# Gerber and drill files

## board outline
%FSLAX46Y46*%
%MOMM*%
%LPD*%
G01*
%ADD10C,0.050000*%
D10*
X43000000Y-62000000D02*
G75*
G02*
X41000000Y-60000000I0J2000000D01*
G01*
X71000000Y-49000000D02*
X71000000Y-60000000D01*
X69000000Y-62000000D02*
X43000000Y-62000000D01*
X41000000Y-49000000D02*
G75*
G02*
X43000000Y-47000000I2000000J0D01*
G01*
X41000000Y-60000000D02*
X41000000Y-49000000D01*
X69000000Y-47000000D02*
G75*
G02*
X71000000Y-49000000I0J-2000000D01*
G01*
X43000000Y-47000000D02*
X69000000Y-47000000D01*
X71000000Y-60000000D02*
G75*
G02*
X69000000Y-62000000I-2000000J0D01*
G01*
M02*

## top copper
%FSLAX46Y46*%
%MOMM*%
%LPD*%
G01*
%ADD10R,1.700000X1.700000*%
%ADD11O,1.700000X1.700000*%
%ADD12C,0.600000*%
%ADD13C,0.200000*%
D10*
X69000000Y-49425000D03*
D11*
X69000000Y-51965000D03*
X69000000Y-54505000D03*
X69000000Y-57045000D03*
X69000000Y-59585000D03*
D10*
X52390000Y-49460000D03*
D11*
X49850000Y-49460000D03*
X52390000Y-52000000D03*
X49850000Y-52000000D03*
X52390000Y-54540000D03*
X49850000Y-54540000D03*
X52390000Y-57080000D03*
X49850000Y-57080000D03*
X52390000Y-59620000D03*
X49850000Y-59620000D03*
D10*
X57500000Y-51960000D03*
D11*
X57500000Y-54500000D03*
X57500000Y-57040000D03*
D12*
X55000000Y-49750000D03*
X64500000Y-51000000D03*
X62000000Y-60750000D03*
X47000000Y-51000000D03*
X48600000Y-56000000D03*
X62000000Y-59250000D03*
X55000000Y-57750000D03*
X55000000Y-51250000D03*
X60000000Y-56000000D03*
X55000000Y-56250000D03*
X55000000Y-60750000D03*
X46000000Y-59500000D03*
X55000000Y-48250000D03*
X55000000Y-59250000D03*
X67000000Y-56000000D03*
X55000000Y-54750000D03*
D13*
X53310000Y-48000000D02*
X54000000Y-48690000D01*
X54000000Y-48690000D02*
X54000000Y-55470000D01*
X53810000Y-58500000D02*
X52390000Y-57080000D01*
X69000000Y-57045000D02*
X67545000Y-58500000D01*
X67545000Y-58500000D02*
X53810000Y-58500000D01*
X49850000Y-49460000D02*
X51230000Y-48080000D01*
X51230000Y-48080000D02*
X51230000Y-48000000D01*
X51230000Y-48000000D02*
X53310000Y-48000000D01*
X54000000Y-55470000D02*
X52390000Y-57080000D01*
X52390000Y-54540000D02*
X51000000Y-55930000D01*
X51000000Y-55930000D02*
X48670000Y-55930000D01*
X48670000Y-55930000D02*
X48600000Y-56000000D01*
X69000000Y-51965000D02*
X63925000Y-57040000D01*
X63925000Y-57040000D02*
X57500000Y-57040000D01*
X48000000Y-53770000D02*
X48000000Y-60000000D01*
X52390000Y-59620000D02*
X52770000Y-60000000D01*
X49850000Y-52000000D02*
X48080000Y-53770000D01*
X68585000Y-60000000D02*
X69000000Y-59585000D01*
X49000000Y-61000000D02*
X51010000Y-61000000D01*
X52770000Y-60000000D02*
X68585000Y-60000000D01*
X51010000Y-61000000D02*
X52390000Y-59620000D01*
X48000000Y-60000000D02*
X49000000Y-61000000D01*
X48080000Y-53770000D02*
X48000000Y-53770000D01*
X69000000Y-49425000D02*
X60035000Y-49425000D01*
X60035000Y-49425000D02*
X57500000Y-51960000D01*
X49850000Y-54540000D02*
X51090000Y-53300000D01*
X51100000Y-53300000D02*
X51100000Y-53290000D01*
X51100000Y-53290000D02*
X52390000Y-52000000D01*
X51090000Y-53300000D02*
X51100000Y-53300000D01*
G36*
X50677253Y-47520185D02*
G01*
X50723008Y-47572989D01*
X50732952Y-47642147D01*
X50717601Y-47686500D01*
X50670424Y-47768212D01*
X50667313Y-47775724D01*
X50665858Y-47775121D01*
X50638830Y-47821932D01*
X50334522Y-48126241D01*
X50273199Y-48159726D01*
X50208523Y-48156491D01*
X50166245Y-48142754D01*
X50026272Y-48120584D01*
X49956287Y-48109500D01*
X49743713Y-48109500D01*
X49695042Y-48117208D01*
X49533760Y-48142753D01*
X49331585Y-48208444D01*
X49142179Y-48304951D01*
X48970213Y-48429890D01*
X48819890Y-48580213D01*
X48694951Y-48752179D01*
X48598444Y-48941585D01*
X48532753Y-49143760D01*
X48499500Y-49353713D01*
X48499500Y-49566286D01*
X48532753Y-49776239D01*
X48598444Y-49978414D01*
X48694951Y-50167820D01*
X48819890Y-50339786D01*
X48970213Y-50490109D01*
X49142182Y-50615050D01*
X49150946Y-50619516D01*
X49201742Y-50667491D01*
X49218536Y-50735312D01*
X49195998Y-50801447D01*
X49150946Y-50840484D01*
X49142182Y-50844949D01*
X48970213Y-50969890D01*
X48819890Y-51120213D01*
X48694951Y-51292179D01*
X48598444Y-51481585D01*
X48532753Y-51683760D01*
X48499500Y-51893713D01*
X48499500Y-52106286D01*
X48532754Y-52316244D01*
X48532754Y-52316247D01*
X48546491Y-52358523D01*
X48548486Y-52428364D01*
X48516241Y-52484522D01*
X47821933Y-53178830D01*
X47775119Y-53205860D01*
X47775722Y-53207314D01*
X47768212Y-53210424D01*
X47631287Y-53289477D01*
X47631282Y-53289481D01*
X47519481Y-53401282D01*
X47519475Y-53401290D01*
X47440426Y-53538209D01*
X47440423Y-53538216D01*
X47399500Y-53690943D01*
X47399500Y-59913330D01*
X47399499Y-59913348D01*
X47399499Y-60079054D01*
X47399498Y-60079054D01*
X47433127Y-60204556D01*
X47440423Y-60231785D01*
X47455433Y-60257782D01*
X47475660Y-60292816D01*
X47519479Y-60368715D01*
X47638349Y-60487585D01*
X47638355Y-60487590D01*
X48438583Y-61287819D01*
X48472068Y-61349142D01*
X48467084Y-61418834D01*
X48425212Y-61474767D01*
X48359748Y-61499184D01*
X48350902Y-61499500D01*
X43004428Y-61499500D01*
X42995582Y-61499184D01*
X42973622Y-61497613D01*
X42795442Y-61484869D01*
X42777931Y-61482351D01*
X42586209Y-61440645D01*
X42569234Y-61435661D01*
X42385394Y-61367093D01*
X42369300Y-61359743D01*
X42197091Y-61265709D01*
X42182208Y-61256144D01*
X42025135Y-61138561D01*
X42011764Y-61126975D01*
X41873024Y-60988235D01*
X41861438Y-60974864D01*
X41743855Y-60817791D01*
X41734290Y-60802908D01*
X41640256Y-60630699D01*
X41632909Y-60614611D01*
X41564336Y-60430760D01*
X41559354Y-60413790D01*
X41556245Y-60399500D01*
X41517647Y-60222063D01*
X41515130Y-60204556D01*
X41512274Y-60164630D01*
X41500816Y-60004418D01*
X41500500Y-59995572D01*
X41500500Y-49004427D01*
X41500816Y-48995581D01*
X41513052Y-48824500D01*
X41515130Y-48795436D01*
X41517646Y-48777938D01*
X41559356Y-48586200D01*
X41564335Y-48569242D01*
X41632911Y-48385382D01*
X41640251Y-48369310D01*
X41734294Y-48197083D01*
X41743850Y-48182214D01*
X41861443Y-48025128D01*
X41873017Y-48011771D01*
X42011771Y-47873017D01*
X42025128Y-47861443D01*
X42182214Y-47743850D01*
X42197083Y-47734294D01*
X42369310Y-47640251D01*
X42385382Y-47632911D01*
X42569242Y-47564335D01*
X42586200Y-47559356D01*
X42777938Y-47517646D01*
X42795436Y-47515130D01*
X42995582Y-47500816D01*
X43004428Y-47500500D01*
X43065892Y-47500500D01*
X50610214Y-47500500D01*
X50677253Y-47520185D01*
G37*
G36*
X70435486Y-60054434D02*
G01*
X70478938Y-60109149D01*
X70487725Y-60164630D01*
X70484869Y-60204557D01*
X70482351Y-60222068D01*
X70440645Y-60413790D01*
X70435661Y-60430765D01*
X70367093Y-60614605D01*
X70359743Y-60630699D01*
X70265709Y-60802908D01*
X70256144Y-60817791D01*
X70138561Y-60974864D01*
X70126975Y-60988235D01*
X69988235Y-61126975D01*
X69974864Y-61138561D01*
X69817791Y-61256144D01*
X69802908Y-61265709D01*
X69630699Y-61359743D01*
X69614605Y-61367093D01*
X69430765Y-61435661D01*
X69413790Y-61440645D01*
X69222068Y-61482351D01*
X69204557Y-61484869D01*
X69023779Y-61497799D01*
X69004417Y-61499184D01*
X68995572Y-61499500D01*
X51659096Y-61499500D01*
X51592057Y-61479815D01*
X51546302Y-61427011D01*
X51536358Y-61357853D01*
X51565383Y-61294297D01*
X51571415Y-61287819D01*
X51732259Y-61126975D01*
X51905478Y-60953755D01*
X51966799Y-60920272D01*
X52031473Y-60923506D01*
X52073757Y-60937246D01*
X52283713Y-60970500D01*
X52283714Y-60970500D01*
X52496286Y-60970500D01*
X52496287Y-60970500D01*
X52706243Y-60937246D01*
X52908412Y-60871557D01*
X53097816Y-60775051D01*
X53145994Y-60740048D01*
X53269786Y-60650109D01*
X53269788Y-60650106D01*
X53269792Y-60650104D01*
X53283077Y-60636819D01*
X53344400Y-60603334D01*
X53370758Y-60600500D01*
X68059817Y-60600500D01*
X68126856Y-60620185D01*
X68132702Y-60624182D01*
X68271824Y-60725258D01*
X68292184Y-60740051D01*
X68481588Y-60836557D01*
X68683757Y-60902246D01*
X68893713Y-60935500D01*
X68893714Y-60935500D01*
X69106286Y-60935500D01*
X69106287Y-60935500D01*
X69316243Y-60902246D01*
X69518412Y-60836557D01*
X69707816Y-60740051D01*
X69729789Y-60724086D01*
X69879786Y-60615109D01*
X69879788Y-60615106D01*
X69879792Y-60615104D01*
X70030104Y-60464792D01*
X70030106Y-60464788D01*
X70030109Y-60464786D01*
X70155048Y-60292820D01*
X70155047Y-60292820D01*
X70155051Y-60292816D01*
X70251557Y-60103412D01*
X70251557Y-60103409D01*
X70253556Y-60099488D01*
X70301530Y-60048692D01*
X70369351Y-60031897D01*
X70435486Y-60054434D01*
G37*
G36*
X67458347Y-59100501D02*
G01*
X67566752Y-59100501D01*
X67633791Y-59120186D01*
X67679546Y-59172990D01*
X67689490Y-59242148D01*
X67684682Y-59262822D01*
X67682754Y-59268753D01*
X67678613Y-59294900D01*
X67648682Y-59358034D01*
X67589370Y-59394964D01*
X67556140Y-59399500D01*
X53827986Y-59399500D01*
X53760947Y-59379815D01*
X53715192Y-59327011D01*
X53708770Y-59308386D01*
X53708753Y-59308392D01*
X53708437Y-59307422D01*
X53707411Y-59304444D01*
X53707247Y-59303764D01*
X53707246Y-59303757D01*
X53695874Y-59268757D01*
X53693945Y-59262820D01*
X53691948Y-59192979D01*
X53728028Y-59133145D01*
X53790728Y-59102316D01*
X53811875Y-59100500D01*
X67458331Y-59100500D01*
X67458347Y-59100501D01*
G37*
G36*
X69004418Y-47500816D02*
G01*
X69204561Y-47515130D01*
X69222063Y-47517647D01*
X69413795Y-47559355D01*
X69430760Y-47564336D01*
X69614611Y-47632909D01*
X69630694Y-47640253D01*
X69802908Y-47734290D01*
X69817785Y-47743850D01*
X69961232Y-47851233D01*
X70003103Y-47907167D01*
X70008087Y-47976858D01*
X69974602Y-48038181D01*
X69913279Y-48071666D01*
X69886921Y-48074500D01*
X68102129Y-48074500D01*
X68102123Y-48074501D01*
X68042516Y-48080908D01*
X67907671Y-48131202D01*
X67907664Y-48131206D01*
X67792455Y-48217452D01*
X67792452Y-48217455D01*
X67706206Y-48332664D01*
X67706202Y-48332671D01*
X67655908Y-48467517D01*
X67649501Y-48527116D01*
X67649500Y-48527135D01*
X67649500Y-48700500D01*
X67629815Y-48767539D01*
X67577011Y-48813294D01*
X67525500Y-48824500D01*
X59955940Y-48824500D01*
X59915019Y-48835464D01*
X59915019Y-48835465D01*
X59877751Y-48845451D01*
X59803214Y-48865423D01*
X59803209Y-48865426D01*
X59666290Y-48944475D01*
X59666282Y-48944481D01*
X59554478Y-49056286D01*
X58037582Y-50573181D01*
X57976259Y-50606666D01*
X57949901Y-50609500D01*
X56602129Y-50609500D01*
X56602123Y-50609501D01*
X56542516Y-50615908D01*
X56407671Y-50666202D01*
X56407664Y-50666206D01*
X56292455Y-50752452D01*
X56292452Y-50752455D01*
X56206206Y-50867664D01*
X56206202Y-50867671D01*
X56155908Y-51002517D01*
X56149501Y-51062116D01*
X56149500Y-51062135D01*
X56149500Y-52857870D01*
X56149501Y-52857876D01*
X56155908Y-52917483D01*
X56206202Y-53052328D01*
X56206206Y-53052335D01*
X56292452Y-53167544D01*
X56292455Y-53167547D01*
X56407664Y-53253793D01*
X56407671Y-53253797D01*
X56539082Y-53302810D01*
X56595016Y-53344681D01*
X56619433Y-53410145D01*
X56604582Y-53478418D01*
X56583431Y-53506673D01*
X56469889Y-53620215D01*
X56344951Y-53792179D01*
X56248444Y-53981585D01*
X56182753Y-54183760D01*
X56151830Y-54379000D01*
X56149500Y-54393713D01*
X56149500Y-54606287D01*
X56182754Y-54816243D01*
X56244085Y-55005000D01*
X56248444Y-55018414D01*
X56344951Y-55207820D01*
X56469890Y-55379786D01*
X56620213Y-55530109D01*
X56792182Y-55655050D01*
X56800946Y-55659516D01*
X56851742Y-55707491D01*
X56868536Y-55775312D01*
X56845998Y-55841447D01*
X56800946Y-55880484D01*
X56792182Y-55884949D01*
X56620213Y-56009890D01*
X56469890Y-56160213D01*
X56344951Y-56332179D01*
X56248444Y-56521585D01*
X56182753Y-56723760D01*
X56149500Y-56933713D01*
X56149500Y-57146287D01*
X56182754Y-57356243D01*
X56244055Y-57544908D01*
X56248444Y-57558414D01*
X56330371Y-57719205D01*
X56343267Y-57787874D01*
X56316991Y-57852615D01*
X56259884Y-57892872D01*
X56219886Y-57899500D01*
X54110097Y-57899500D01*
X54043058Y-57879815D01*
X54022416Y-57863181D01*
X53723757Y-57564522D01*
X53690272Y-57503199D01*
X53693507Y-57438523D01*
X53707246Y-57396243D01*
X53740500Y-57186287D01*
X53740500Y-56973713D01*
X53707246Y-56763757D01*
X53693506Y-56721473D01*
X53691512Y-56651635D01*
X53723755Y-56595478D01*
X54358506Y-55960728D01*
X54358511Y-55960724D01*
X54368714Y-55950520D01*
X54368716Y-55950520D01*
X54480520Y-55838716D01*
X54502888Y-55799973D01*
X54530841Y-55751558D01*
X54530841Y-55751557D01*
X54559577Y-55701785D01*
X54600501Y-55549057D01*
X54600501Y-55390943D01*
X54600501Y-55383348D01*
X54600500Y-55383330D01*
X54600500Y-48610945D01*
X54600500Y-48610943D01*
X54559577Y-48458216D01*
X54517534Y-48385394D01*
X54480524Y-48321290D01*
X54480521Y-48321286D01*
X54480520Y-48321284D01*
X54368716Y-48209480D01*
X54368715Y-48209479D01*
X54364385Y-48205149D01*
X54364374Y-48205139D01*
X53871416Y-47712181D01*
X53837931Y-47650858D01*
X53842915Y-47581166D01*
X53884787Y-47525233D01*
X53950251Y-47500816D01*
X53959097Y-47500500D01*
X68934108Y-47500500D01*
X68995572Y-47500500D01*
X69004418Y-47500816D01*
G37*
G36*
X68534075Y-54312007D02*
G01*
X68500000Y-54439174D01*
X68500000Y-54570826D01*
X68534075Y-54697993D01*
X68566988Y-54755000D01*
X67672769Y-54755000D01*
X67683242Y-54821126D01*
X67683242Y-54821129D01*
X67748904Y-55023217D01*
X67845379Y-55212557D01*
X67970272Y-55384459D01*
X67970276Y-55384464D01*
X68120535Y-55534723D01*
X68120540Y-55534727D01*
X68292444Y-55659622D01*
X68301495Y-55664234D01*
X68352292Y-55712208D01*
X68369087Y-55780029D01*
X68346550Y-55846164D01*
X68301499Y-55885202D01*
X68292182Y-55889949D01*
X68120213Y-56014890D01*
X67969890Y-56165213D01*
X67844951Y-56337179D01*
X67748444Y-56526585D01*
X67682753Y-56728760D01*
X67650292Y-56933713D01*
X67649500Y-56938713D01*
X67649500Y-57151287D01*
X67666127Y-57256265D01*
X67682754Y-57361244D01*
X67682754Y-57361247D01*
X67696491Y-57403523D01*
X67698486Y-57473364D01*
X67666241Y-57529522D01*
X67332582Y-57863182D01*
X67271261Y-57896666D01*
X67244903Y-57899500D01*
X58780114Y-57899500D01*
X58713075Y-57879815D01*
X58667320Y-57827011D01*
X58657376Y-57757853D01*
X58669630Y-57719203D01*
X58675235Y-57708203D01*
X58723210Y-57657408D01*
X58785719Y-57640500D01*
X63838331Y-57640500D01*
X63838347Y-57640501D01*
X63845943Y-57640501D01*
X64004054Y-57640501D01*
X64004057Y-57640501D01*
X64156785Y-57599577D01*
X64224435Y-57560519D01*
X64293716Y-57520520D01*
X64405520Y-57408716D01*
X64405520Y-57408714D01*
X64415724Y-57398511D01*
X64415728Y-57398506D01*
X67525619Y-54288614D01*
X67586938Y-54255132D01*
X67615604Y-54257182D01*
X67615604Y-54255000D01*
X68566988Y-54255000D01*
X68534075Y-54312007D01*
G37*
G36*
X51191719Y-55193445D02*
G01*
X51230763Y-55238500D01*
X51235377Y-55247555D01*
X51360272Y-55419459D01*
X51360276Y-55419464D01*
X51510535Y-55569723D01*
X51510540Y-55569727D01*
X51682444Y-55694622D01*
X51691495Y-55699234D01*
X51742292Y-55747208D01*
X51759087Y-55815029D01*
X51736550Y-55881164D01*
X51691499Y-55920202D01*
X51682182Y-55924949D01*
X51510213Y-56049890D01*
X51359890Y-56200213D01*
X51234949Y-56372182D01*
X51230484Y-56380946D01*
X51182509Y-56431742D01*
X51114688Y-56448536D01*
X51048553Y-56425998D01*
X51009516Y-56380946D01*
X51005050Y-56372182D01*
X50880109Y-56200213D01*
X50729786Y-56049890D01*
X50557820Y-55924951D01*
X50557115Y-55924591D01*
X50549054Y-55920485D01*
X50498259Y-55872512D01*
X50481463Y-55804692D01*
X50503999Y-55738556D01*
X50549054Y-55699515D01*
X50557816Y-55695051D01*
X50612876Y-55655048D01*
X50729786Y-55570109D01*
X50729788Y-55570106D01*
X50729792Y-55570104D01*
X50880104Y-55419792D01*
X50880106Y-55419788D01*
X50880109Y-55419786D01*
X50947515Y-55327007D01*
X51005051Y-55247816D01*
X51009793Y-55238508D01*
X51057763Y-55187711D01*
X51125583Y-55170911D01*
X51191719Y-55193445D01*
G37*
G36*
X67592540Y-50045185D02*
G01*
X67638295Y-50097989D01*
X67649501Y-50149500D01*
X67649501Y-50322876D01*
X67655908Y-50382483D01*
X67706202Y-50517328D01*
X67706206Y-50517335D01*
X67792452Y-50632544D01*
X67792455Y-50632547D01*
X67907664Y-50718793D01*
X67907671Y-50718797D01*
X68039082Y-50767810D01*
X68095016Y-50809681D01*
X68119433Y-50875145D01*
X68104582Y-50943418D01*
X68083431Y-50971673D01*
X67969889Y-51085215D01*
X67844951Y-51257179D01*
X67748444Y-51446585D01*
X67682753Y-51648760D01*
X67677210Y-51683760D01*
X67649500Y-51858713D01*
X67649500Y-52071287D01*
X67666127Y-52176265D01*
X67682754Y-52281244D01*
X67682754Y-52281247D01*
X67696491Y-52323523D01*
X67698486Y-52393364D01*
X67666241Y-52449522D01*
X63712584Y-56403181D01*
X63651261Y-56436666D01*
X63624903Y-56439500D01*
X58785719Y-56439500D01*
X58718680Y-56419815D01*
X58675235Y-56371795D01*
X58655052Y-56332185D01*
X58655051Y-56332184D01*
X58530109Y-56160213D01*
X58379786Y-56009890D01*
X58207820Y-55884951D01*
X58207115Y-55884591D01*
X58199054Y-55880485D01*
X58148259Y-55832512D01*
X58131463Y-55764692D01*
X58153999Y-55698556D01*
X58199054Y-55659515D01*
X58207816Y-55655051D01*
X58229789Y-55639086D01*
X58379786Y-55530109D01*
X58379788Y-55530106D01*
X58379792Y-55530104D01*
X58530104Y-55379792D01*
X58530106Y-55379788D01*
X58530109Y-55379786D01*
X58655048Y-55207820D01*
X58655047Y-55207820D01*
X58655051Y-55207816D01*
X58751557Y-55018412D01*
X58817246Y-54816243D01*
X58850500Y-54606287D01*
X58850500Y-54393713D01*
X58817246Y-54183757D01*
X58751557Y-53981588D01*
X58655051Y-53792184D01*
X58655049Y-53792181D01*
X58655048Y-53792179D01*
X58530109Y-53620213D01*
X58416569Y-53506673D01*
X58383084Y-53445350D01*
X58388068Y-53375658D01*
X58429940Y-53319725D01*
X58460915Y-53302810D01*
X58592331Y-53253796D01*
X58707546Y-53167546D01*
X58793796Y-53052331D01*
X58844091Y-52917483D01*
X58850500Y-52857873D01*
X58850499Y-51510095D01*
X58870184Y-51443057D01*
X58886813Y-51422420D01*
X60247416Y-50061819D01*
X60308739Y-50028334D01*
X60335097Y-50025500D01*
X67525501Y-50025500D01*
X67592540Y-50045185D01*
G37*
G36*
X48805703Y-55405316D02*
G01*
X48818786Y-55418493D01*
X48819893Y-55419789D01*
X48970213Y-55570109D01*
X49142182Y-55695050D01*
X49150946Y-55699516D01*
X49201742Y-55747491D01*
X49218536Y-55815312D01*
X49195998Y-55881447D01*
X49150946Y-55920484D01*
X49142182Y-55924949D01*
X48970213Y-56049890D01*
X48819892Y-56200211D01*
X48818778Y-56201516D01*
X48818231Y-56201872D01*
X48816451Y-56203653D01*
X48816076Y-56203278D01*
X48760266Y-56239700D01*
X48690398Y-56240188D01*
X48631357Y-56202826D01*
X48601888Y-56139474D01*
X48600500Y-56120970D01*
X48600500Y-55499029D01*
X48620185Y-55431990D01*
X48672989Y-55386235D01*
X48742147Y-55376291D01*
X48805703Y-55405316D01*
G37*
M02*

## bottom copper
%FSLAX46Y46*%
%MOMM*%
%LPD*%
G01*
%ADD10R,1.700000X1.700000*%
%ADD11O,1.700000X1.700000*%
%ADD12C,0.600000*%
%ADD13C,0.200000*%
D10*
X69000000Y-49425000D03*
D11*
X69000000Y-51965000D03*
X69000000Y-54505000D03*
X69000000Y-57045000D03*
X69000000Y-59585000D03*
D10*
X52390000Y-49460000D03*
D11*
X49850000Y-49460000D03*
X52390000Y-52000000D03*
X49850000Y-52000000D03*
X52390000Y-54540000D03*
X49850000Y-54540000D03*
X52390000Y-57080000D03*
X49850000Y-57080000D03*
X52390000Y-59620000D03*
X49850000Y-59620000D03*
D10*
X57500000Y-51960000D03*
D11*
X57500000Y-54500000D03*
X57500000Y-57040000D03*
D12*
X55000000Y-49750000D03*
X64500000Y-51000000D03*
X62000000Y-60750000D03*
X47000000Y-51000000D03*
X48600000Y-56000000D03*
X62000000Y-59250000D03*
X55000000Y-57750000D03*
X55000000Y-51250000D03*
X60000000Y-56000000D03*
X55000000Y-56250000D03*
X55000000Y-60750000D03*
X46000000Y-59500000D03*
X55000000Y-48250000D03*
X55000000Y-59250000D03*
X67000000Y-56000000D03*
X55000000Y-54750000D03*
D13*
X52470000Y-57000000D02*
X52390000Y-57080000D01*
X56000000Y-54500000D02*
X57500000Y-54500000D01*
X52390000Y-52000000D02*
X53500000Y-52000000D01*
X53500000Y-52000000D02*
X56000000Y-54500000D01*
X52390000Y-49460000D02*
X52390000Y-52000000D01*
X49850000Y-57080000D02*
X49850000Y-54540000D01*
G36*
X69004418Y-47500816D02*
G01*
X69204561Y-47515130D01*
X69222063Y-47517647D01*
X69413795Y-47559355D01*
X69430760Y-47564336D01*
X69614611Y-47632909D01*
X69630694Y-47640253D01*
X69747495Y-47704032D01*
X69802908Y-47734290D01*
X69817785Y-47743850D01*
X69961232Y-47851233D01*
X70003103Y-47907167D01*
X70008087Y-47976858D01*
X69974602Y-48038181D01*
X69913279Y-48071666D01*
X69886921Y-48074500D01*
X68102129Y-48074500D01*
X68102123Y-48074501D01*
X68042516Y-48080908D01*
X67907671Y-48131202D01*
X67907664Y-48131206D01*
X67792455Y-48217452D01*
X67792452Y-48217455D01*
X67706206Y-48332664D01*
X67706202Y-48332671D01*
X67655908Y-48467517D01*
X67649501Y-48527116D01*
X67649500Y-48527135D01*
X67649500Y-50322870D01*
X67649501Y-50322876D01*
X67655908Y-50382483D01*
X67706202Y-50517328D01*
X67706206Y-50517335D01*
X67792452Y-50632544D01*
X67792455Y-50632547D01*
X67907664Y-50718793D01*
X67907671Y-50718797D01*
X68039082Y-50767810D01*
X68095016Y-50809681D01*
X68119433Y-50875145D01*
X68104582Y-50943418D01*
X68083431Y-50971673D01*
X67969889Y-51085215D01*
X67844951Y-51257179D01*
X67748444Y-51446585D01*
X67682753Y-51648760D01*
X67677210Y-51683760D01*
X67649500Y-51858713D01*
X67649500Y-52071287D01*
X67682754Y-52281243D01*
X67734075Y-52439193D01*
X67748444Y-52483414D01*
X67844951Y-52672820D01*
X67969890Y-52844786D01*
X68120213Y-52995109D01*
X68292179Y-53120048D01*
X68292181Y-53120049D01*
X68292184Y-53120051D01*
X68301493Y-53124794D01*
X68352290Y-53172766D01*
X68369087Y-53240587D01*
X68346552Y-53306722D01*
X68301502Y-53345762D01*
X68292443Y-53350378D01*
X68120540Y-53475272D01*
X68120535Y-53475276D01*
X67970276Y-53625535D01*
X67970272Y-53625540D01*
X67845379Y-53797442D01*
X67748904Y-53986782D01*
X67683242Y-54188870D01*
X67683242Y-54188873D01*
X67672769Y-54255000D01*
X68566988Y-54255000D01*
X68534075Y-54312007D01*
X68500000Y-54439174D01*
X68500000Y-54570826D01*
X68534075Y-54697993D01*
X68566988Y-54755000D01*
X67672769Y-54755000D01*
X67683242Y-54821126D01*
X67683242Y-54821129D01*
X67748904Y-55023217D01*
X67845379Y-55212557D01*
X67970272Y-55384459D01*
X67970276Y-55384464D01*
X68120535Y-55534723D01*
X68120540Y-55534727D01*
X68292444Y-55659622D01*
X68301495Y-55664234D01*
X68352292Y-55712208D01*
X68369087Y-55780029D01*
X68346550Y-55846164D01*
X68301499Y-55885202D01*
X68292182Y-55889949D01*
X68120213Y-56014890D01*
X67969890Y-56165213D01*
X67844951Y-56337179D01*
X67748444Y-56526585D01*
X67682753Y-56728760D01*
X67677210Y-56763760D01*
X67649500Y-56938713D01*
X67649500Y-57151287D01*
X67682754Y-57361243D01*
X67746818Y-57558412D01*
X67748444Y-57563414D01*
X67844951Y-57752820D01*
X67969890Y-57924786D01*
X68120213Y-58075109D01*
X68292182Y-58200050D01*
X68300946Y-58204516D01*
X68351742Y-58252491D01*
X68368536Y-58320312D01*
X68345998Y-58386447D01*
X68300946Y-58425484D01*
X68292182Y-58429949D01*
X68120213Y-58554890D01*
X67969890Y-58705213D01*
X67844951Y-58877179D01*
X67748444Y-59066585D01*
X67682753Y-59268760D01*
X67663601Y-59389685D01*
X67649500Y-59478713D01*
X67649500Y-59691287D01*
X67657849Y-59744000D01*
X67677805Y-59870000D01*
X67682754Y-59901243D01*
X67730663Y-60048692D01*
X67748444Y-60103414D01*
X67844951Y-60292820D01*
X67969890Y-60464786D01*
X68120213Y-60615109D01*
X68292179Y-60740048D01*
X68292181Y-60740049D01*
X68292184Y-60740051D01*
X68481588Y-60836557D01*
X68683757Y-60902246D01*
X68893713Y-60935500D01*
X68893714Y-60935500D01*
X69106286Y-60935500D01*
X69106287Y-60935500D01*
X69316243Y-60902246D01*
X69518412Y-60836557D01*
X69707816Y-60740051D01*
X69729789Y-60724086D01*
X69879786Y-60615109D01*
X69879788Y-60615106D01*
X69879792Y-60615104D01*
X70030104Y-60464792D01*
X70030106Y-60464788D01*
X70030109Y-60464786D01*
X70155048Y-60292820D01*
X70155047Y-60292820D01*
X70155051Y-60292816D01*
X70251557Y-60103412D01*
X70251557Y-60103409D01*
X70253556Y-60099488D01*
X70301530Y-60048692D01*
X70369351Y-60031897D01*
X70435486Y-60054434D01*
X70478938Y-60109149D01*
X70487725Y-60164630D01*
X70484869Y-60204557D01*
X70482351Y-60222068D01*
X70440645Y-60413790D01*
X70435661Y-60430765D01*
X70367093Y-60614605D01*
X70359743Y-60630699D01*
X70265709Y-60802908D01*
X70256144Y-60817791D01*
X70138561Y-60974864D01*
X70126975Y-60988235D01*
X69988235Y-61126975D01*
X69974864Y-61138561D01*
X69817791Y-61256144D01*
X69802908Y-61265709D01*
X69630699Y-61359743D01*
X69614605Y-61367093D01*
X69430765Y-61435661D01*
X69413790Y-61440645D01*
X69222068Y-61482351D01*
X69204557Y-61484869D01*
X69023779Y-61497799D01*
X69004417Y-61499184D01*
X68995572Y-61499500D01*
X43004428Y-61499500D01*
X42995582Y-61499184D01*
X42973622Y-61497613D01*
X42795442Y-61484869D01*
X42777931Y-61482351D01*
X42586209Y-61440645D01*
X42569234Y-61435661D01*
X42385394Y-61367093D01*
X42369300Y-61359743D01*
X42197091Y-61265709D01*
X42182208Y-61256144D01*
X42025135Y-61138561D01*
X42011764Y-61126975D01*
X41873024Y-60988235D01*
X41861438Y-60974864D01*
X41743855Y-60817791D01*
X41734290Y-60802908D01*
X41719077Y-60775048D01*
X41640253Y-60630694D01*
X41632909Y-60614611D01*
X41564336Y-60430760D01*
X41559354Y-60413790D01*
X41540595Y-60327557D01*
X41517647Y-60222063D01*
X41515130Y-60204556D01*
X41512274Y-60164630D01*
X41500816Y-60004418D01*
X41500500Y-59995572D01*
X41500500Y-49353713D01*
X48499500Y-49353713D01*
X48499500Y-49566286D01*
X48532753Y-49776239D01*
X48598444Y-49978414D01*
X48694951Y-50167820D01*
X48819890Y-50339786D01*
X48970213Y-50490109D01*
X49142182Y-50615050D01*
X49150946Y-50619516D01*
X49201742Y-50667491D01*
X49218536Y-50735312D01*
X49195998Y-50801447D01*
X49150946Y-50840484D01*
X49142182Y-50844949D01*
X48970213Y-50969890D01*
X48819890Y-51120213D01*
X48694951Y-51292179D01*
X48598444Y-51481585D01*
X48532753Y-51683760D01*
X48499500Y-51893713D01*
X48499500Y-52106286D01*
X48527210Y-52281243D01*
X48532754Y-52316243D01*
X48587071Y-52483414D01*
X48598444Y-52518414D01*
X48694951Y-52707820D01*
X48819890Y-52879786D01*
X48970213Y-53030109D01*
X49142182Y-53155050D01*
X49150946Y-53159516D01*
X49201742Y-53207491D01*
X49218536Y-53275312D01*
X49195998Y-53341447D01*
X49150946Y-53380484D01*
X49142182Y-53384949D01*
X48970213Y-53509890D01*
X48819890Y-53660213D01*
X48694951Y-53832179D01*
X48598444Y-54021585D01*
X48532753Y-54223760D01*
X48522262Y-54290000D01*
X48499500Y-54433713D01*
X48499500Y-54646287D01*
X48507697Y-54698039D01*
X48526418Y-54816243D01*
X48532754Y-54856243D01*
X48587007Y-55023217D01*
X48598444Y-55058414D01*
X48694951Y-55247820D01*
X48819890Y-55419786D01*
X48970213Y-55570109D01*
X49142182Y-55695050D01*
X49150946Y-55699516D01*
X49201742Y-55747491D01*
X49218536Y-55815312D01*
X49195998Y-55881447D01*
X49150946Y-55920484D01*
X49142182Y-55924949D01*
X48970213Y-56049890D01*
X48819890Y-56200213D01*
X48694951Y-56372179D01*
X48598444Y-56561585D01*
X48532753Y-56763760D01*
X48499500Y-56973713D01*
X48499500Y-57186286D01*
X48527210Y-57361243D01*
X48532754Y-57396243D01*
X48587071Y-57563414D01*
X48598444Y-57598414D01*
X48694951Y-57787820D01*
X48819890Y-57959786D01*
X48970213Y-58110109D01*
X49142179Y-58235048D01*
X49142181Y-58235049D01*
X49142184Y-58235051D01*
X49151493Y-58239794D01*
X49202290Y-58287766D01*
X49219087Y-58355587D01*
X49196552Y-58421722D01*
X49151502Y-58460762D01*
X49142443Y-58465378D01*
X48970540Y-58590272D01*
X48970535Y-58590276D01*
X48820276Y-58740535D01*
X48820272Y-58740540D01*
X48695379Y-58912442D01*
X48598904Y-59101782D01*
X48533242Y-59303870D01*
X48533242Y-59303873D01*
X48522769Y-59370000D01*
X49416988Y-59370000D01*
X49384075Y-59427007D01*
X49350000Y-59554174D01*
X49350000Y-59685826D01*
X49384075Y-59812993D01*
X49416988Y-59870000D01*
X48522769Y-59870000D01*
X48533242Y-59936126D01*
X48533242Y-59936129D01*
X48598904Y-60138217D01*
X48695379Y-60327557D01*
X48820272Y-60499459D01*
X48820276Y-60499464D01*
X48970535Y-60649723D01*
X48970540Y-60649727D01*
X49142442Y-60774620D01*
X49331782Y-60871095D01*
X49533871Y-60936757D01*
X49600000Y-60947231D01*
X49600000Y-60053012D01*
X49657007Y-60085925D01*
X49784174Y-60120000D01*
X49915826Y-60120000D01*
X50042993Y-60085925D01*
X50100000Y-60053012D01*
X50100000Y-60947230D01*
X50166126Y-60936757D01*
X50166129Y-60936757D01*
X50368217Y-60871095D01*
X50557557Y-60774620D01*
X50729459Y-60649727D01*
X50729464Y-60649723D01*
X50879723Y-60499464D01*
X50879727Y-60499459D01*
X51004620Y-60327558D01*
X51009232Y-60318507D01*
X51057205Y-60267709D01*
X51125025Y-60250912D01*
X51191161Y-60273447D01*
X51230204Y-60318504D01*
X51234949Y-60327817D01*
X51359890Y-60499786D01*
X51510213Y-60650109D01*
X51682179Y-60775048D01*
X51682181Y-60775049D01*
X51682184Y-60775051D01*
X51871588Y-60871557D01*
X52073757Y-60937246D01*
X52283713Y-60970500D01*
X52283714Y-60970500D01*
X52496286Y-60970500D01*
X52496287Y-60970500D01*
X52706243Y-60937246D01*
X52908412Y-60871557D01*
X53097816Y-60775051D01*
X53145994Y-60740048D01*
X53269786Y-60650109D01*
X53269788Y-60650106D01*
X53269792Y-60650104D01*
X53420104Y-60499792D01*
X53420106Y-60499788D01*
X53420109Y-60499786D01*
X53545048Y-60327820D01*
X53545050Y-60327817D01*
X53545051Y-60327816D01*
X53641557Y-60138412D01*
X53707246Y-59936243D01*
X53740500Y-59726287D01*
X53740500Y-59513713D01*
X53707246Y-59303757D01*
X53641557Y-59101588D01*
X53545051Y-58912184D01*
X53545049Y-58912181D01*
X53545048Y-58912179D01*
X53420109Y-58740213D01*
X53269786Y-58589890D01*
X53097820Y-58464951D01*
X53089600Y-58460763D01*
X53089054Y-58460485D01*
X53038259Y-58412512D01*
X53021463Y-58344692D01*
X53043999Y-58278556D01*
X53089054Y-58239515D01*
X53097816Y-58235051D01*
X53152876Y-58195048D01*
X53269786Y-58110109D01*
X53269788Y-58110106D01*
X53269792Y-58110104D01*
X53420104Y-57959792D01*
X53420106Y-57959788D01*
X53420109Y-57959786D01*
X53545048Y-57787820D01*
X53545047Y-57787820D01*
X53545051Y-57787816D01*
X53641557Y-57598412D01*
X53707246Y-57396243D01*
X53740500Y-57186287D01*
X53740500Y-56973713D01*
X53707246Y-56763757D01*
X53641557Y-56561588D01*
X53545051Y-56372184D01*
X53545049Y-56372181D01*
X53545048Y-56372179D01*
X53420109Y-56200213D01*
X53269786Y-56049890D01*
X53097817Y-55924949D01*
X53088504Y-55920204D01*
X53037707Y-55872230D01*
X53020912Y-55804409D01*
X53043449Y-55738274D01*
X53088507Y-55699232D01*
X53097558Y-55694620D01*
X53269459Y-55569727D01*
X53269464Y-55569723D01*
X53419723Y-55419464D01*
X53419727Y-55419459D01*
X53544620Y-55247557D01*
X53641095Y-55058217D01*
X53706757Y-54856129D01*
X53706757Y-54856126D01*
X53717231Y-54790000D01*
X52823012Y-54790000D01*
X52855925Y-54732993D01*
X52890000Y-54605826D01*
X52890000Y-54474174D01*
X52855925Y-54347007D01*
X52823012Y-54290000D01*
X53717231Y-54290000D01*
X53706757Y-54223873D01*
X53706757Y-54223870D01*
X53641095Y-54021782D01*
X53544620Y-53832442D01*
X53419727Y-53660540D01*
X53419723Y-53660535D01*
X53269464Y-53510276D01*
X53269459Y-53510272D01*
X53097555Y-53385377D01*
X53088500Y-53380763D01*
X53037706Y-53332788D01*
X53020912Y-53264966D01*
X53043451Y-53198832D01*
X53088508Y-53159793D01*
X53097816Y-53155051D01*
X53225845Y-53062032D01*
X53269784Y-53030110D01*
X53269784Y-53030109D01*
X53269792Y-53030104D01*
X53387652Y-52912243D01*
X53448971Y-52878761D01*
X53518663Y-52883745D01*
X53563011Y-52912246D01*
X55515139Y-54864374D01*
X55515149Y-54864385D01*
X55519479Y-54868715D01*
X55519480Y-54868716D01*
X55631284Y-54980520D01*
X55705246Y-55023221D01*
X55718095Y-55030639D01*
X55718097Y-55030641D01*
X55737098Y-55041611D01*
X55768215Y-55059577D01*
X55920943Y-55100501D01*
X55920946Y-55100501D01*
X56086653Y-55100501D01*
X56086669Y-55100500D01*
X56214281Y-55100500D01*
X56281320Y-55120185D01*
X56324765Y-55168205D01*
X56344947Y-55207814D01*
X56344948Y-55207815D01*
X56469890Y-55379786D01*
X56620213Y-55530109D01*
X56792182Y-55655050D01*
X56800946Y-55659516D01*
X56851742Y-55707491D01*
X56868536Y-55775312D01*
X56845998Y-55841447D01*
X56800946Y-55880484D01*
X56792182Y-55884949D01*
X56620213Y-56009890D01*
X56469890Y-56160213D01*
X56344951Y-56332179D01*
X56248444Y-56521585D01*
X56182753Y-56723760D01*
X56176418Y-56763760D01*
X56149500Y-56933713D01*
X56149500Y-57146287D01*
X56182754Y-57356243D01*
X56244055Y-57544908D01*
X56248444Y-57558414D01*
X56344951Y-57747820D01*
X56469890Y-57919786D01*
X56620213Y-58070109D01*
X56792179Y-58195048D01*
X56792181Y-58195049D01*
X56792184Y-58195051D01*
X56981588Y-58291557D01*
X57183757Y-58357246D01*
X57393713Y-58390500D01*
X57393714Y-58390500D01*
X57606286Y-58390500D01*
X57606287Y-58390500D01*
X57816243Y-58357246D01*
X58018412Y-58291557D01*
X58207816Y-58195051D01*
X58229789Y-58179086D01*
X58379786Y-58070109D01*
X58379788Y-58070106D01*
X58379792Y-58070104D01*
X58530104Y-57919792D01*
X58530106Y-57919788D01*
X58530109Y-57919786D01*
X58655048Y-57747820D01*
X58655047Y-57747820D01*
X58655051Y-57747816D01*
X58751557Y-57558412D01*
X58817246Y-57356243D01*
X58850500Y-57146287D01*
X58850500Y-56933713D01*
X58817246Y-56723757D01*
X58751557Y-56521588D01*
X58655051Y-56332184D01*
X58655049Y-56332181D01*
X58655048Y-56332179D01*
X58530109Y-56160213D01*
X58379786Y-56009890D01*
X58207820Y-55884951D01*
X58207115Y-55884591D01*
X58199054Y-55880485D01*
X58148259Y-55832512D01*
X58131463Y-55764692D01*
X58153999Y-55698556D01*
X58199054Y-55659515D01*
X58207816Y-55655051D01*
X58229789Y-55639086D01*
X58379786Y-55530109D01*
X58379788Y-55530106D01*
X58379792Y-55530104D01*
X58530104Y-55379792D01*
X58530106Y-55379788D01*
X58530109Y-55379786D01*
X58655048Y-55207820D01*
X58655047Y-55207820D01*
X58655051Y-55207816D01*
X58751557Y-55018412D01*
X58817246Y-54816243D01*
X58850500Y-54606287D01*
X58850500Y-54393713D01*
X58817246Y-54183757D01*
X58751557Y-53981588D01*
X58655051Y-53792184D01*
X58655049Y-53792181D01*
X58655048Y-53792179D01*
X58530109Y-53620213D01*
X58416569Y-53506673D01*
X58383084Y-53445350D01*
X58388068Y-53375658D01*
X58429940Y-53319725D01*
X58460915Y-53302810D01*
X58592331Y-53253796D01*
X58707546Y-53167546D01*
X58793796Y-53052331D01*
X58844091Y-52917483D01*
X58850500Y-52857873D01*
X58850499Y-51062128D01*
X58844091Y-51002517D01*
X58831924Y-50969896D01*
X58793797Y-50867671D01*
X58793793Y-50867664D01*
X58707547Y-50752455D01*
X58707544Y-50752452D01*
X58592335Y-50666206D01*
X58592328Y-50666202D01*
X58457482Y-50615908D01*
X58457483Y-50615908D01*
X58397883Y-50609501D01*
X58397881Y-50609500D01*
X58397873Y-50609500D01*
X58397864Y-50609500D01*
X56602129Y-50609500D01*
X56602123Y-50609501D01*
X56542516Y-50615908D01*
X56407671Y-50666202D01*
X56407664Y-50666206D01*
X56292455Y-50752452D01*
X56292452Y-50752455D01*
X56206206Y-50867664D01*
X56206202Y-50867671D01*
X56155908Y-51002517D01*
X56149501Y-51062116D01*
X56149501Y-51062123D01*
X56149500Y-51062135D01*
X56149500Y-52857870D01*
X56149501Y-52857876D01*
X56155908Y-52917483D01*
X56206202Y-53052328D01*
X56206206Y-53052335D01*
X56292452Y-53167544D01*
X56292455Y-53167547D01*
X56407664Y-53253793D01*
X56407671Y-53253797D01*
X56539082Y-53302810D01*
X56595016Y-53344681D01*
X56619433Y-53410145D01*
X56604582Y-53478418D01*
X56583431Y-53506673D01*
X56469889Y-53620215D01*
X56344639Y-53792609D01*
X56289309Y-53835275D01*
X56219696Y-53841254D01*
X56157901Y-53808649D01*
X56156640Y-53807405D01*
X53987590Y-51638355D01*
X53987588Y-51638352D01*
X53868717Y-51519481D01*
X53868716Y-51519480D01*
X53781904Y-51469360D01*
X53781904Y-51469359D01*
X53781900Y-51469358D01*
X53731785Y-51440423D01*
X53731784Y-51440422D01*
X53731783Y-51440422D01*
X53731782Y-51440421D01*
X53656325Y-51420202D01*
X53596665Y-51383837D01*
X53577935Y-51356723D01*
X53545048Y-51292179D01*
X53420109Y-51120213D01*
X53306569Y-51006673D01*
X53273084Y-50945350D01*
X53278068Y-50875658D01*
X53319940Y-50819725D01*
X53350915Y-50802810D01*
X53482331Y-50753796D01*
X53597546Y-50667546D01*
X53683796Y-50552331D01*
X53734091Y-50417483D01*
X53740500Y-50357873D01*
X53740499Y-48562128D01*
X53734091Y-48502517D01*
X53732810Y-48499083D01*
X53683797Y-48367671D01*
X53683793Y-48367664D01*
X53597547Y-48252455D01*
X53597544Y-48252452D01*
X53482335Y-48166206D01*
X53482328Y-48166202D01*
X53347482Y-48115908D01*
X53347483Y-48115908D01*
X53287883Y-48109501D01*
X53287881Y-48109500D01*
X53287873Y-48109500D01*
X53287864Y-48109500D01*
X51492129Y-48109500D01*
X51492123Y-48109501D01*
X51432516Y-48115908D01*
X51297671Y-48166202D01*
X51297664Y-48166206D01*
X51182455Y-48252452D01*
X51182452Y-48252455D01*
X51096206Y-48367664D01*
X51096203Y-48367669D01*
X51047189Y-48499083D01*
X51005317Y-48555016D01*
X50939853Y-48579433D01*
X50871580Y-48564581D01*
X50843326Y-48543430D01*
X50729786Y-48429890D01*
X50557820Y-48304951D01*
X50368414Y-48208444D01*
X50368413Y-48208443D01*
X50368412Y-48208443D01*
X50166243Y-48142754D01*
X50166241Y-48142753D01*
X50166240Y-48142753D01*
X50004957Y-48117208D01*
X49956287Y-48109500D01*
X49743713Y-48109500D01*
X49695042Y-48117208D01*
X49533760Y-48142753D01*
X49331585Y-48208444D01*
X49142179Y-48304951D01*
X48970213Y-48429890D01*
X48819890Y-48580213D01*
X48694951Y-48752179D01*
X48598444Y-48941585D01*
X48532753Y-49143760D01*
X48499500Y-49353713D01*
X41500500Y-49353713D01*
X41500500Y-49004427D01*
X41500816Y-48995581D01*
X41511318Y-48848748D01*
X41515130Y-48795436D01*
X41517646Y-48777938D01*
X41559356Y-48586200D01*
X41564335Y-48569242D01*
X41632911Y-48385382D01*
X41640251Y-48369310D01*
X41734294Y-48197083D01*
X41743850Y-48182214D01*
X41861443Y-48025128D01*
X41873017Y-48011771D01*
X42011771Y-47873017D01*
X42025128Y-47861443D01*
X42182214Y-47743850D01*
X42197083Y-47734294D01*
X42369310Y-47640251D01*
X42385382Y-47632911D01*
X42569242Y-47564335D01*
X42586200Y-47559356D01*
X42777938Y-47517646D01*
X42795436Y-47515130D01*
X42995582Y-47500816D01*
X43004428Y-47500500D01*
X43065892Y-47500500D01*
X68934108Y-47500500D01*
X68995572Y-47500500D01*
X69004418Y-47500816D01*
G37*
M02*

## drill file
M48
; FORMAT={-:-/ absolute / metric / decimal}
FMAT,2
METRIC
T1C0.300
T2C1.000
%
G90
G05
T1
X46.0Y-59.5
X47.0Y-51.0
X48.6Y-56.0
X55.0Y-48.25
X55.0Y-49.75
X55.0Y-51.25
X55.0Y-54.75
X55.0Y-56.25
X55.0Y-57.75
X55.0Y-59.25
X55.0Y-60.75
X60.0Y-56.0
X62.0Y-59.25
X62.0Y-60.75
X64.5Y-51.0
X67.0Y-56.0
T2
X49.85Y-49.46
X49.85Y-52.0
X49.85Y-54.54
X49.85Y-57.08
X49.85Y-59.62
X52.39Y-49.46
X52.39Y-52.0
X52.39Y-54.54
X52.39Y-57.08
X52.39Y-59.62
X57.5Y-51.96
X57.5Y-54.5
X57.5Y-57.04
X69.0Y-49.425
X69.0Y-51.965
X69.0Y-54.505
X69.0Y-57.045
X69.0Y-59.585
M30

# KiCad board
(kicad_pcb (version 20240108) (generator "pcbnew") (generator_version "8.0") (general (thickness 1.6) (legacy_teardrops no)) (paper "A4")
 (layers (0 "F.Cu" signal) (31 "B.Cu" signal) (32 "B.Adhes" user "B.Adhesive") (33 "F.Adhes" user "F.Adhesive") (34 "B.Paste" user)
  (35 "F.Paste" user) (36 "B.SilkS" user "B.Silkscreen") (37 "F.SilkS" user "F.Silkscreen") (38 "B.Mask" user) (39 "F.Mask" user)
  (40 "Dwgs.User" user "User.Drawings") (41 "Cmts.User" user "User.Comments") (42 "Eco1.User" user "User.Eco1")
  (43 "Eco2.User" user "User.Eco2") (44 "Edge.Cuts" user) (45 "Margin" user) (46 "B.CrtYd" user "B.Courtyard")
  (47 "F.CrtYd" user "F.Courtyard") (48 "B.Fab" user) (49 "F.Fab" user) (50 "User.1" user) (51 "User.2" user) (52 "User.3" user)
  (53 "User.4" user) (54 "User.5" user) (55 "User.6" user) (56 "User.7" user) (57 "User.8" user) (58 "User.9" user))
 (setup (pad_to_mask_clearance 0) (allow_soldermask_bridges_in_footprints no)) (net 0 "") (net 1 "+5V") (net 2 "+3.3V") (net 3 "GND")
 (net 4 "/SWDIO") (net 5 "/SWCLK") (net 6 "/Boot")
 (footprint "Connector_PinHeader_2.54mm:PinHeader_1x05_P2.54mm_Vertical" (layer "F.Cu") (at 69 49.425)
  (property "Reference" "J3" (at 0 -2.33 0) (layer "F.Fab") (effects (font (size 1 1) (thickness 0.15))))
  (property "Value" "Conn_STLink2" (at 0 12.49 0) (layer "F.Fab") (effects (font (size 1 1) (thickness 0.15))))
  (pad "1" thru_hole rect (at 0 0) (size 1.7 1.7) (drill 1) (layers "*.Cu" "*.Mask") (remove_unused_layers no) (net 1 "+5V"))
  (pad "2" thru_hole oval (at 0 2.54) (size 1.7 1.7) (drill 1) (layers "*.Cu" "*.Mask") (remove_unused_layers no) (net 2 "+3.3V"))
  (pad "3" thru_hole oval (at 0 5.08) (size 1.7 1.7) (drill 1) (layers "*.Cu" "*.Mask") (remove_unused_layers no) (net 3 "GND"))
  (pad "4" thru_hole oval (at 0 7.62) (size 1.7 1.7) (drill 1) (layers "*.Cu" "*.Mask") (remove_unused_layers no) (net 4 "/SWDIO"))
  (pad "5" thru_hole oval (at 0 10.16) (size 1.7 1.7) (drill 1) (layers "*.Cu" "*.Mask") (remove_unused_layers no) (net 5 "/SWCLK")))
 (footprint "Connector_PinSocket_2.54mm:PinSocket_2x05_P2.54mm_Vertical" (layer "F.Cu") (at 52.39 49.46)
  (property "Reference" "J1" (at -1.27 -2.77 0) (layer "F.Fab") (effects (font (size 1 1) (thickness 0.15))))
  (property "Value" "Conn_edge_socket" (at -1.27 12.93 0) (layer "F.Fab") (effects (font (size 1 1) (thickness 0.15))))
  (pad "1" thru_hole rect (at 0 0) (size 1.7 1.7) (drill 1) (layers "*.Cu" "*.Mask") (remove_unused_layers no) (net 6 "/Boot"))
  (pad "2" thru_hole oval (at -2.54 0) (size 1.7 1.7) (drill 1) (layers "*.Cu" "*.Mask") (remove_unused_layers no) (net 4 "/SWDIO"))
  (pad "3" thru_hole oval (at 0 2.54) (size 1.7 1.7) (drill 1) (layers "*.Cu" "*.Mask") (remove_unused_layers no) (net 6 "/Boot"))
  (pad "4" thru_hole oval (at -2.54 2.54) (size 1.7 1.7) (drill 1) (layers "*.Cu" "*.Mask") (remove_unused_layers no) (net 5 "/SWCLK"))
  (pad "5" thru_hole oval (at 0 5.08) (size 1.7 1.7) (drill 1) (layers "*.Cu" "*.Mask") (remove_unused_layers no) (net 3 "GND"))
  (pad "6" thru_hole oval (at -2.54 5.08) (size 1.7 1.7) (drill 1) (layers "*.Cu" "*.Mask") (remove_unused_layers no) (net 6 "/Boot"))
  (pad "7" thru_hole oval (at 0 7.62) (size 1.7 1.7) (drill 1) (layers "*.Cu" "*.Mask") (remove_unused_layers no) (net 4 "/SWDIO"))
  (pad "8" thru_hole oval (at -2.54 7.62) (size 1.7 1.7) (drill 1) (layers "*.Cu" "*.Mask") (remove_unused_layers no) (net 6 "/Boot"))
  (pad "9" thru_hole oval (at 0 10.16) (size 1.7 1.7) (drill 1) (layers "*.Cu" "*.Mask") (remove_unused_layers no) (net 5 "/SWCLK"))
  (pad "10" thru_hole oval (at -2.54 10.16) (size 1.7 1.7) (drill 1) (layers "*.Cu" "*.Mask") (remove_unused_layers no) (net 3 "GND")))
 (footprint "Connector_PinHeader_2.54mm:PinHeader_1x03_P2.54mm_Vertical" (layer "F.Cu") (at 57.5 51.96)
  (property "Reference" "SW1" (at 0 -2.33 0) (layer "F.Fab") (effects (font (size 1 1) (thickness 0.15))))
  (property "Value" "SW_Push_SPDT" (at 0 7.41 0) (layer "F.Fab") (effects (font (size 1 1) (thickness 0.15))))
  (pad "1" thru_hole rect (at 0 0) (size 1.7 1.7) (drill 1) (layers "*.Cu" "*.Mask") (remove_unused_layers no) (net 1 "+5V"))
  (pad "2" thru_hole oval (at 0 2.54) (size 1.7 1.7) (drill 1) (layers "*.Cu" "*.Mask") (remove_unused_layers no) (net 6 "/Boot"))
  (pad "3" thru_hole oval (at 0 5.08) (size 1.7 1.7) (drill 1) (layers "*.Cu" "*.Mask") (remove_unused_layers no) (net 2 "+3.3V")))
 (gr_arc (start 43 62) (mid 41.585786 61.414214) (end 41 60) (stroke (width 0.05) (type default)) (layer "Edge.Cuts"))
 (gr_line (start 71 49) (end 71 60) (stroke (width 0.05) (type default)) (layer "Edge.Cuts"))
 (gr_line (start 69 62) (end 43 62) (stroke (width 0.05) (type default)) (layer "Edge.Cuts"))
 (gr_arc (start 41 49) (mid 41.585786 47.585786) (end 43 47) (stroke (width 0.05) (type default)) (layer "Edge.Cuts"))
 (gr_line (start 41 60) (end 41 49) (stroke (width 0.05) (type default)) (layer "Edge.Cuts"))
 (gr_arc (start 69 47) (mid 70.414214 47.585786) (end 71 49) (stroke (width 0.05) (type default)) (layer "Edge.Cuts"))
 (gr_line (start 43 47) (end 69 47) (stroke (width 0.05) (type default)) (layer "Edge.Cuts"))
 (gr_arc (start 71 60) (mid 70.414214 61.414214) (end 69 62) (stroke (width 0.05) (type default)) (layer "Edge.Cuts"))
 (segment (start 53.31 48) (end 54 48.69) (width 0.2) (layer "F.Cu") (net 4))
 (segment (start 54 48.69) (end 54 55.47) (width 0.2) (layer "F.Cu") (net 4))
 (segment (start 53.81 58.5) (end 52.39 57.08) (width 0.2) (layer "F.Cu") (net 4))
 (segment (start 69 57.045) (end 67.545 58.5) (width 0.2) (layer "F.Cu") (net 4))
 (segment (start 67.545 58.5) (end 53.81 58.5) (width 0.2) (layer "F.Cu") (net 4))
 (segment (start 49.85 49.46) (end 51.23 48.08) (width 0.2) (layer "F.Cu") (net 4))
 (segment (start 51.23 48.08) (end 51.23 48) (width 0.2) (layer "F.Cu") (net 4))
 (segment (start 51.23 48) (end 53.31 48) (width 0.2) (layer "F.Cu") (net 4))
 (segment (start 54 55.47) (end 52.39 57.08) (width 0.2) (layer "F.Cu") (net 4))
 (segment (start 52.47 57) (end 52.39 57.08) (width 0.2) (layer "B.Cu") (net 4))
 (segment (start 52.39 54.54) (end 51 55.93) (width 0.2) (layer "F.Cu") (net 3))
 (segment (start 51 55.93) (end 48.67 55.93) (width 0.2) (layer "F.Cu") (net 3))
 (segment (start 48.67 55.93) (end 48.6 56) (width 0.2) (layer "F.Cu") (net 3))
 (via (at 55 49.75) (size 0.6) (drill 0.3) (layers "F.Cu" "B.Cu") (free yes) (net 3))
 (via (at 64.5 51) (size 0.6) (drill 0.3) (layers "F.Cu" "B.Cu") (free yes) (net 3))
 (via (at 62 60.75) (size 0.6) (drill 0.3) (layers "F.Cu" "B.Cu") (free yes) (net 3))
 (via (at 47 51) (size 0.6) (drill 0.3) (layers "F.Cu" "B.Cu") (free yes) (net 3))
 (via (at 48.6 56) (size 0.6) (drill 0.3) (layers "F.Cu" "B.Cu") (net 3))
 (via (at 62 59.25) (size 0.6) (drill 0.3) (layers "F.Cu" "B.Cu") (free yes) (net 3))
 (via (at 55 57.75) (size 0.6) (drill 0.3) (layers "F.Cu" "B.Cu") (free yes) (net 3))
 (via (at 55 51.25) (size 0.6) (drill 0.3) (layers "F.Cu" "B.Cu") (free yes) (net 3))
 (via (at 60 56) (size 0.6) (drill 0.3) (layers "F.Cu" "B.Cu") (free yes) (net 3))
 (via (at 55 56.25) (size 0.6) (drill 0.3) (layers "F.Cu" "B.Cu") (free yes) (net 3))
 (via (at 55 60.75) (size 0.6) (drill 0.3) (layers "F.Cu" "B.Cu") (free yes) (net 3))
 (via (at 46 59.5) (size 0.6) (drill 0.3) (layers "F.Cu" "B.Cu") (free yes) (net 3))
 (via (at 55 48.25) (size 0.6) (drill 0.3) (layers "F.Cu" "B.Cu") (free yes) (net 3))
 (via (at 55 59.25) (size 0.6) (drill 0.3) (layers "F.Cu" "B.Cu") (free yes) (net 3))
 (via (at 67 56) (size 0.6) (drill 0.3) (layers "F.Cu" "B.Cu") (free yes) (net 3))
 (via (at 55 54.75) (size 0.6) (drill 0.3) (layers "F.Cu" "B.Cu") (free yes) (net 3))
 (segment (start 69 51.965) (end 63.925 57.04) (width 0.2) (layer "F.Cu") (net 2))
 (segment (start 63.925 57.04) (end 57.5 57.04) (width 0.2) (layer "F.Cu") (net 2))
 (segment (start 48 53.77) (end 48 60) (width 0.2) (layer "F.Cu") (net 5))
 (segment (start 52.39 59.62) (end 52.77 60) (width 0.2) (layer "F.Cu") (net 5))
 (segment (start 49.85 52) (end 48.08 53.77) (width 0.2) (layer "F.Cu") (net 5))
 (segment (start 68.585 60) (end 69 59.585) (width 0.2) (layer "F.Cu") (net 5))
 (segment (start 49 61) (end 51.01 61) (width 0.2) (layer "F.Cu") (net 5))
 (segment (start 52.77 60) (end 68.585 60) (width 0.2) (layer "F.Cu") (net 5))
 (segment (start 51.01 61) (end 52.39 59.62) (width 0.2) (layer "F.Cu") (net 5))
 (segment (start 48 60) (end 49 61) (width 0.2) (layer "F.Cu") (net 5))
 (segment (start 48.08 53.77) (end 48 53.77) (width 0.2) (layer "F.Cu") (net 5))
 (segment (start 69 49.425) (end 60.035 49.425) (width 0.2) (layer "F.Cu") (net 1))
 (segment (start 60.035 49.425) (end 57.5 51.96) (width 0.2) (layer "F.Cu") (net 1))
 (segment (start 49.85 54.54) (end 51.09 53.3) (width 0.2) (layer "F.Cu") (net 6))
 (segment (start 51.1 53.3) (end 51.1 53.29) (width 0.2) (layer "F.Cu") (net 6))
 (segment (start 51.1 53.29) (end 52.39 52) (width 0.2) (layer "F.Cu") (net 6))
 (segment (start 51.09 53.3) (end 51.1 53.3) (width 0.2) (layer "F.Cu") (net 6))
 (segment (start 56 54.5) (end 57.5 54.5) (width 0.2) (layer "B.Cu") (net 6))
 (segment (start 52.39 52) (end 53.5 52) (width 0.2) (layer "B.Cu") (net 6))
 (segment (start 53.5 52) (end 56 54.5) (width 0.2) (layer "B.Cu") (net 6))
 (segment (start 52.39 49.46) (end 52.39 52) (width 0.2) (layer "B.Cu") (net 6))
 (segment (start 49.85 57.08) (end 49.85 54.54) (width 0.2) (layer "B.Cu") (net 6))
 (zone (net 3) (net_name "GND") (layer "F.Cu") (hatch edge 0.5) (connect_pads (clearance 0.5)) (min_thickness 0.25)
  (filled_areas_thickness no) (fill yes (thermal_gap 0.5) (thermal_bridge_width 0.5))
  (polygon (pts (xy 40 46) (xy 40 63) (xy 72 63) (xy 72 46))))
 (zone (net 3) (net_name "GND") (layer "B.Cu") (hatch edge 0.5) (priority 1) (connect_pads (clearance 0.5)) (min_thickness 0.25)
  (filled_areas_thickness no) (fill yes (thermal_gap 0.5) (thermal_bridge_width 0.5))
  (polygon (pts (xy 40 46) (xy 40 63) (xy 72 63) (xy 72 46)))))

